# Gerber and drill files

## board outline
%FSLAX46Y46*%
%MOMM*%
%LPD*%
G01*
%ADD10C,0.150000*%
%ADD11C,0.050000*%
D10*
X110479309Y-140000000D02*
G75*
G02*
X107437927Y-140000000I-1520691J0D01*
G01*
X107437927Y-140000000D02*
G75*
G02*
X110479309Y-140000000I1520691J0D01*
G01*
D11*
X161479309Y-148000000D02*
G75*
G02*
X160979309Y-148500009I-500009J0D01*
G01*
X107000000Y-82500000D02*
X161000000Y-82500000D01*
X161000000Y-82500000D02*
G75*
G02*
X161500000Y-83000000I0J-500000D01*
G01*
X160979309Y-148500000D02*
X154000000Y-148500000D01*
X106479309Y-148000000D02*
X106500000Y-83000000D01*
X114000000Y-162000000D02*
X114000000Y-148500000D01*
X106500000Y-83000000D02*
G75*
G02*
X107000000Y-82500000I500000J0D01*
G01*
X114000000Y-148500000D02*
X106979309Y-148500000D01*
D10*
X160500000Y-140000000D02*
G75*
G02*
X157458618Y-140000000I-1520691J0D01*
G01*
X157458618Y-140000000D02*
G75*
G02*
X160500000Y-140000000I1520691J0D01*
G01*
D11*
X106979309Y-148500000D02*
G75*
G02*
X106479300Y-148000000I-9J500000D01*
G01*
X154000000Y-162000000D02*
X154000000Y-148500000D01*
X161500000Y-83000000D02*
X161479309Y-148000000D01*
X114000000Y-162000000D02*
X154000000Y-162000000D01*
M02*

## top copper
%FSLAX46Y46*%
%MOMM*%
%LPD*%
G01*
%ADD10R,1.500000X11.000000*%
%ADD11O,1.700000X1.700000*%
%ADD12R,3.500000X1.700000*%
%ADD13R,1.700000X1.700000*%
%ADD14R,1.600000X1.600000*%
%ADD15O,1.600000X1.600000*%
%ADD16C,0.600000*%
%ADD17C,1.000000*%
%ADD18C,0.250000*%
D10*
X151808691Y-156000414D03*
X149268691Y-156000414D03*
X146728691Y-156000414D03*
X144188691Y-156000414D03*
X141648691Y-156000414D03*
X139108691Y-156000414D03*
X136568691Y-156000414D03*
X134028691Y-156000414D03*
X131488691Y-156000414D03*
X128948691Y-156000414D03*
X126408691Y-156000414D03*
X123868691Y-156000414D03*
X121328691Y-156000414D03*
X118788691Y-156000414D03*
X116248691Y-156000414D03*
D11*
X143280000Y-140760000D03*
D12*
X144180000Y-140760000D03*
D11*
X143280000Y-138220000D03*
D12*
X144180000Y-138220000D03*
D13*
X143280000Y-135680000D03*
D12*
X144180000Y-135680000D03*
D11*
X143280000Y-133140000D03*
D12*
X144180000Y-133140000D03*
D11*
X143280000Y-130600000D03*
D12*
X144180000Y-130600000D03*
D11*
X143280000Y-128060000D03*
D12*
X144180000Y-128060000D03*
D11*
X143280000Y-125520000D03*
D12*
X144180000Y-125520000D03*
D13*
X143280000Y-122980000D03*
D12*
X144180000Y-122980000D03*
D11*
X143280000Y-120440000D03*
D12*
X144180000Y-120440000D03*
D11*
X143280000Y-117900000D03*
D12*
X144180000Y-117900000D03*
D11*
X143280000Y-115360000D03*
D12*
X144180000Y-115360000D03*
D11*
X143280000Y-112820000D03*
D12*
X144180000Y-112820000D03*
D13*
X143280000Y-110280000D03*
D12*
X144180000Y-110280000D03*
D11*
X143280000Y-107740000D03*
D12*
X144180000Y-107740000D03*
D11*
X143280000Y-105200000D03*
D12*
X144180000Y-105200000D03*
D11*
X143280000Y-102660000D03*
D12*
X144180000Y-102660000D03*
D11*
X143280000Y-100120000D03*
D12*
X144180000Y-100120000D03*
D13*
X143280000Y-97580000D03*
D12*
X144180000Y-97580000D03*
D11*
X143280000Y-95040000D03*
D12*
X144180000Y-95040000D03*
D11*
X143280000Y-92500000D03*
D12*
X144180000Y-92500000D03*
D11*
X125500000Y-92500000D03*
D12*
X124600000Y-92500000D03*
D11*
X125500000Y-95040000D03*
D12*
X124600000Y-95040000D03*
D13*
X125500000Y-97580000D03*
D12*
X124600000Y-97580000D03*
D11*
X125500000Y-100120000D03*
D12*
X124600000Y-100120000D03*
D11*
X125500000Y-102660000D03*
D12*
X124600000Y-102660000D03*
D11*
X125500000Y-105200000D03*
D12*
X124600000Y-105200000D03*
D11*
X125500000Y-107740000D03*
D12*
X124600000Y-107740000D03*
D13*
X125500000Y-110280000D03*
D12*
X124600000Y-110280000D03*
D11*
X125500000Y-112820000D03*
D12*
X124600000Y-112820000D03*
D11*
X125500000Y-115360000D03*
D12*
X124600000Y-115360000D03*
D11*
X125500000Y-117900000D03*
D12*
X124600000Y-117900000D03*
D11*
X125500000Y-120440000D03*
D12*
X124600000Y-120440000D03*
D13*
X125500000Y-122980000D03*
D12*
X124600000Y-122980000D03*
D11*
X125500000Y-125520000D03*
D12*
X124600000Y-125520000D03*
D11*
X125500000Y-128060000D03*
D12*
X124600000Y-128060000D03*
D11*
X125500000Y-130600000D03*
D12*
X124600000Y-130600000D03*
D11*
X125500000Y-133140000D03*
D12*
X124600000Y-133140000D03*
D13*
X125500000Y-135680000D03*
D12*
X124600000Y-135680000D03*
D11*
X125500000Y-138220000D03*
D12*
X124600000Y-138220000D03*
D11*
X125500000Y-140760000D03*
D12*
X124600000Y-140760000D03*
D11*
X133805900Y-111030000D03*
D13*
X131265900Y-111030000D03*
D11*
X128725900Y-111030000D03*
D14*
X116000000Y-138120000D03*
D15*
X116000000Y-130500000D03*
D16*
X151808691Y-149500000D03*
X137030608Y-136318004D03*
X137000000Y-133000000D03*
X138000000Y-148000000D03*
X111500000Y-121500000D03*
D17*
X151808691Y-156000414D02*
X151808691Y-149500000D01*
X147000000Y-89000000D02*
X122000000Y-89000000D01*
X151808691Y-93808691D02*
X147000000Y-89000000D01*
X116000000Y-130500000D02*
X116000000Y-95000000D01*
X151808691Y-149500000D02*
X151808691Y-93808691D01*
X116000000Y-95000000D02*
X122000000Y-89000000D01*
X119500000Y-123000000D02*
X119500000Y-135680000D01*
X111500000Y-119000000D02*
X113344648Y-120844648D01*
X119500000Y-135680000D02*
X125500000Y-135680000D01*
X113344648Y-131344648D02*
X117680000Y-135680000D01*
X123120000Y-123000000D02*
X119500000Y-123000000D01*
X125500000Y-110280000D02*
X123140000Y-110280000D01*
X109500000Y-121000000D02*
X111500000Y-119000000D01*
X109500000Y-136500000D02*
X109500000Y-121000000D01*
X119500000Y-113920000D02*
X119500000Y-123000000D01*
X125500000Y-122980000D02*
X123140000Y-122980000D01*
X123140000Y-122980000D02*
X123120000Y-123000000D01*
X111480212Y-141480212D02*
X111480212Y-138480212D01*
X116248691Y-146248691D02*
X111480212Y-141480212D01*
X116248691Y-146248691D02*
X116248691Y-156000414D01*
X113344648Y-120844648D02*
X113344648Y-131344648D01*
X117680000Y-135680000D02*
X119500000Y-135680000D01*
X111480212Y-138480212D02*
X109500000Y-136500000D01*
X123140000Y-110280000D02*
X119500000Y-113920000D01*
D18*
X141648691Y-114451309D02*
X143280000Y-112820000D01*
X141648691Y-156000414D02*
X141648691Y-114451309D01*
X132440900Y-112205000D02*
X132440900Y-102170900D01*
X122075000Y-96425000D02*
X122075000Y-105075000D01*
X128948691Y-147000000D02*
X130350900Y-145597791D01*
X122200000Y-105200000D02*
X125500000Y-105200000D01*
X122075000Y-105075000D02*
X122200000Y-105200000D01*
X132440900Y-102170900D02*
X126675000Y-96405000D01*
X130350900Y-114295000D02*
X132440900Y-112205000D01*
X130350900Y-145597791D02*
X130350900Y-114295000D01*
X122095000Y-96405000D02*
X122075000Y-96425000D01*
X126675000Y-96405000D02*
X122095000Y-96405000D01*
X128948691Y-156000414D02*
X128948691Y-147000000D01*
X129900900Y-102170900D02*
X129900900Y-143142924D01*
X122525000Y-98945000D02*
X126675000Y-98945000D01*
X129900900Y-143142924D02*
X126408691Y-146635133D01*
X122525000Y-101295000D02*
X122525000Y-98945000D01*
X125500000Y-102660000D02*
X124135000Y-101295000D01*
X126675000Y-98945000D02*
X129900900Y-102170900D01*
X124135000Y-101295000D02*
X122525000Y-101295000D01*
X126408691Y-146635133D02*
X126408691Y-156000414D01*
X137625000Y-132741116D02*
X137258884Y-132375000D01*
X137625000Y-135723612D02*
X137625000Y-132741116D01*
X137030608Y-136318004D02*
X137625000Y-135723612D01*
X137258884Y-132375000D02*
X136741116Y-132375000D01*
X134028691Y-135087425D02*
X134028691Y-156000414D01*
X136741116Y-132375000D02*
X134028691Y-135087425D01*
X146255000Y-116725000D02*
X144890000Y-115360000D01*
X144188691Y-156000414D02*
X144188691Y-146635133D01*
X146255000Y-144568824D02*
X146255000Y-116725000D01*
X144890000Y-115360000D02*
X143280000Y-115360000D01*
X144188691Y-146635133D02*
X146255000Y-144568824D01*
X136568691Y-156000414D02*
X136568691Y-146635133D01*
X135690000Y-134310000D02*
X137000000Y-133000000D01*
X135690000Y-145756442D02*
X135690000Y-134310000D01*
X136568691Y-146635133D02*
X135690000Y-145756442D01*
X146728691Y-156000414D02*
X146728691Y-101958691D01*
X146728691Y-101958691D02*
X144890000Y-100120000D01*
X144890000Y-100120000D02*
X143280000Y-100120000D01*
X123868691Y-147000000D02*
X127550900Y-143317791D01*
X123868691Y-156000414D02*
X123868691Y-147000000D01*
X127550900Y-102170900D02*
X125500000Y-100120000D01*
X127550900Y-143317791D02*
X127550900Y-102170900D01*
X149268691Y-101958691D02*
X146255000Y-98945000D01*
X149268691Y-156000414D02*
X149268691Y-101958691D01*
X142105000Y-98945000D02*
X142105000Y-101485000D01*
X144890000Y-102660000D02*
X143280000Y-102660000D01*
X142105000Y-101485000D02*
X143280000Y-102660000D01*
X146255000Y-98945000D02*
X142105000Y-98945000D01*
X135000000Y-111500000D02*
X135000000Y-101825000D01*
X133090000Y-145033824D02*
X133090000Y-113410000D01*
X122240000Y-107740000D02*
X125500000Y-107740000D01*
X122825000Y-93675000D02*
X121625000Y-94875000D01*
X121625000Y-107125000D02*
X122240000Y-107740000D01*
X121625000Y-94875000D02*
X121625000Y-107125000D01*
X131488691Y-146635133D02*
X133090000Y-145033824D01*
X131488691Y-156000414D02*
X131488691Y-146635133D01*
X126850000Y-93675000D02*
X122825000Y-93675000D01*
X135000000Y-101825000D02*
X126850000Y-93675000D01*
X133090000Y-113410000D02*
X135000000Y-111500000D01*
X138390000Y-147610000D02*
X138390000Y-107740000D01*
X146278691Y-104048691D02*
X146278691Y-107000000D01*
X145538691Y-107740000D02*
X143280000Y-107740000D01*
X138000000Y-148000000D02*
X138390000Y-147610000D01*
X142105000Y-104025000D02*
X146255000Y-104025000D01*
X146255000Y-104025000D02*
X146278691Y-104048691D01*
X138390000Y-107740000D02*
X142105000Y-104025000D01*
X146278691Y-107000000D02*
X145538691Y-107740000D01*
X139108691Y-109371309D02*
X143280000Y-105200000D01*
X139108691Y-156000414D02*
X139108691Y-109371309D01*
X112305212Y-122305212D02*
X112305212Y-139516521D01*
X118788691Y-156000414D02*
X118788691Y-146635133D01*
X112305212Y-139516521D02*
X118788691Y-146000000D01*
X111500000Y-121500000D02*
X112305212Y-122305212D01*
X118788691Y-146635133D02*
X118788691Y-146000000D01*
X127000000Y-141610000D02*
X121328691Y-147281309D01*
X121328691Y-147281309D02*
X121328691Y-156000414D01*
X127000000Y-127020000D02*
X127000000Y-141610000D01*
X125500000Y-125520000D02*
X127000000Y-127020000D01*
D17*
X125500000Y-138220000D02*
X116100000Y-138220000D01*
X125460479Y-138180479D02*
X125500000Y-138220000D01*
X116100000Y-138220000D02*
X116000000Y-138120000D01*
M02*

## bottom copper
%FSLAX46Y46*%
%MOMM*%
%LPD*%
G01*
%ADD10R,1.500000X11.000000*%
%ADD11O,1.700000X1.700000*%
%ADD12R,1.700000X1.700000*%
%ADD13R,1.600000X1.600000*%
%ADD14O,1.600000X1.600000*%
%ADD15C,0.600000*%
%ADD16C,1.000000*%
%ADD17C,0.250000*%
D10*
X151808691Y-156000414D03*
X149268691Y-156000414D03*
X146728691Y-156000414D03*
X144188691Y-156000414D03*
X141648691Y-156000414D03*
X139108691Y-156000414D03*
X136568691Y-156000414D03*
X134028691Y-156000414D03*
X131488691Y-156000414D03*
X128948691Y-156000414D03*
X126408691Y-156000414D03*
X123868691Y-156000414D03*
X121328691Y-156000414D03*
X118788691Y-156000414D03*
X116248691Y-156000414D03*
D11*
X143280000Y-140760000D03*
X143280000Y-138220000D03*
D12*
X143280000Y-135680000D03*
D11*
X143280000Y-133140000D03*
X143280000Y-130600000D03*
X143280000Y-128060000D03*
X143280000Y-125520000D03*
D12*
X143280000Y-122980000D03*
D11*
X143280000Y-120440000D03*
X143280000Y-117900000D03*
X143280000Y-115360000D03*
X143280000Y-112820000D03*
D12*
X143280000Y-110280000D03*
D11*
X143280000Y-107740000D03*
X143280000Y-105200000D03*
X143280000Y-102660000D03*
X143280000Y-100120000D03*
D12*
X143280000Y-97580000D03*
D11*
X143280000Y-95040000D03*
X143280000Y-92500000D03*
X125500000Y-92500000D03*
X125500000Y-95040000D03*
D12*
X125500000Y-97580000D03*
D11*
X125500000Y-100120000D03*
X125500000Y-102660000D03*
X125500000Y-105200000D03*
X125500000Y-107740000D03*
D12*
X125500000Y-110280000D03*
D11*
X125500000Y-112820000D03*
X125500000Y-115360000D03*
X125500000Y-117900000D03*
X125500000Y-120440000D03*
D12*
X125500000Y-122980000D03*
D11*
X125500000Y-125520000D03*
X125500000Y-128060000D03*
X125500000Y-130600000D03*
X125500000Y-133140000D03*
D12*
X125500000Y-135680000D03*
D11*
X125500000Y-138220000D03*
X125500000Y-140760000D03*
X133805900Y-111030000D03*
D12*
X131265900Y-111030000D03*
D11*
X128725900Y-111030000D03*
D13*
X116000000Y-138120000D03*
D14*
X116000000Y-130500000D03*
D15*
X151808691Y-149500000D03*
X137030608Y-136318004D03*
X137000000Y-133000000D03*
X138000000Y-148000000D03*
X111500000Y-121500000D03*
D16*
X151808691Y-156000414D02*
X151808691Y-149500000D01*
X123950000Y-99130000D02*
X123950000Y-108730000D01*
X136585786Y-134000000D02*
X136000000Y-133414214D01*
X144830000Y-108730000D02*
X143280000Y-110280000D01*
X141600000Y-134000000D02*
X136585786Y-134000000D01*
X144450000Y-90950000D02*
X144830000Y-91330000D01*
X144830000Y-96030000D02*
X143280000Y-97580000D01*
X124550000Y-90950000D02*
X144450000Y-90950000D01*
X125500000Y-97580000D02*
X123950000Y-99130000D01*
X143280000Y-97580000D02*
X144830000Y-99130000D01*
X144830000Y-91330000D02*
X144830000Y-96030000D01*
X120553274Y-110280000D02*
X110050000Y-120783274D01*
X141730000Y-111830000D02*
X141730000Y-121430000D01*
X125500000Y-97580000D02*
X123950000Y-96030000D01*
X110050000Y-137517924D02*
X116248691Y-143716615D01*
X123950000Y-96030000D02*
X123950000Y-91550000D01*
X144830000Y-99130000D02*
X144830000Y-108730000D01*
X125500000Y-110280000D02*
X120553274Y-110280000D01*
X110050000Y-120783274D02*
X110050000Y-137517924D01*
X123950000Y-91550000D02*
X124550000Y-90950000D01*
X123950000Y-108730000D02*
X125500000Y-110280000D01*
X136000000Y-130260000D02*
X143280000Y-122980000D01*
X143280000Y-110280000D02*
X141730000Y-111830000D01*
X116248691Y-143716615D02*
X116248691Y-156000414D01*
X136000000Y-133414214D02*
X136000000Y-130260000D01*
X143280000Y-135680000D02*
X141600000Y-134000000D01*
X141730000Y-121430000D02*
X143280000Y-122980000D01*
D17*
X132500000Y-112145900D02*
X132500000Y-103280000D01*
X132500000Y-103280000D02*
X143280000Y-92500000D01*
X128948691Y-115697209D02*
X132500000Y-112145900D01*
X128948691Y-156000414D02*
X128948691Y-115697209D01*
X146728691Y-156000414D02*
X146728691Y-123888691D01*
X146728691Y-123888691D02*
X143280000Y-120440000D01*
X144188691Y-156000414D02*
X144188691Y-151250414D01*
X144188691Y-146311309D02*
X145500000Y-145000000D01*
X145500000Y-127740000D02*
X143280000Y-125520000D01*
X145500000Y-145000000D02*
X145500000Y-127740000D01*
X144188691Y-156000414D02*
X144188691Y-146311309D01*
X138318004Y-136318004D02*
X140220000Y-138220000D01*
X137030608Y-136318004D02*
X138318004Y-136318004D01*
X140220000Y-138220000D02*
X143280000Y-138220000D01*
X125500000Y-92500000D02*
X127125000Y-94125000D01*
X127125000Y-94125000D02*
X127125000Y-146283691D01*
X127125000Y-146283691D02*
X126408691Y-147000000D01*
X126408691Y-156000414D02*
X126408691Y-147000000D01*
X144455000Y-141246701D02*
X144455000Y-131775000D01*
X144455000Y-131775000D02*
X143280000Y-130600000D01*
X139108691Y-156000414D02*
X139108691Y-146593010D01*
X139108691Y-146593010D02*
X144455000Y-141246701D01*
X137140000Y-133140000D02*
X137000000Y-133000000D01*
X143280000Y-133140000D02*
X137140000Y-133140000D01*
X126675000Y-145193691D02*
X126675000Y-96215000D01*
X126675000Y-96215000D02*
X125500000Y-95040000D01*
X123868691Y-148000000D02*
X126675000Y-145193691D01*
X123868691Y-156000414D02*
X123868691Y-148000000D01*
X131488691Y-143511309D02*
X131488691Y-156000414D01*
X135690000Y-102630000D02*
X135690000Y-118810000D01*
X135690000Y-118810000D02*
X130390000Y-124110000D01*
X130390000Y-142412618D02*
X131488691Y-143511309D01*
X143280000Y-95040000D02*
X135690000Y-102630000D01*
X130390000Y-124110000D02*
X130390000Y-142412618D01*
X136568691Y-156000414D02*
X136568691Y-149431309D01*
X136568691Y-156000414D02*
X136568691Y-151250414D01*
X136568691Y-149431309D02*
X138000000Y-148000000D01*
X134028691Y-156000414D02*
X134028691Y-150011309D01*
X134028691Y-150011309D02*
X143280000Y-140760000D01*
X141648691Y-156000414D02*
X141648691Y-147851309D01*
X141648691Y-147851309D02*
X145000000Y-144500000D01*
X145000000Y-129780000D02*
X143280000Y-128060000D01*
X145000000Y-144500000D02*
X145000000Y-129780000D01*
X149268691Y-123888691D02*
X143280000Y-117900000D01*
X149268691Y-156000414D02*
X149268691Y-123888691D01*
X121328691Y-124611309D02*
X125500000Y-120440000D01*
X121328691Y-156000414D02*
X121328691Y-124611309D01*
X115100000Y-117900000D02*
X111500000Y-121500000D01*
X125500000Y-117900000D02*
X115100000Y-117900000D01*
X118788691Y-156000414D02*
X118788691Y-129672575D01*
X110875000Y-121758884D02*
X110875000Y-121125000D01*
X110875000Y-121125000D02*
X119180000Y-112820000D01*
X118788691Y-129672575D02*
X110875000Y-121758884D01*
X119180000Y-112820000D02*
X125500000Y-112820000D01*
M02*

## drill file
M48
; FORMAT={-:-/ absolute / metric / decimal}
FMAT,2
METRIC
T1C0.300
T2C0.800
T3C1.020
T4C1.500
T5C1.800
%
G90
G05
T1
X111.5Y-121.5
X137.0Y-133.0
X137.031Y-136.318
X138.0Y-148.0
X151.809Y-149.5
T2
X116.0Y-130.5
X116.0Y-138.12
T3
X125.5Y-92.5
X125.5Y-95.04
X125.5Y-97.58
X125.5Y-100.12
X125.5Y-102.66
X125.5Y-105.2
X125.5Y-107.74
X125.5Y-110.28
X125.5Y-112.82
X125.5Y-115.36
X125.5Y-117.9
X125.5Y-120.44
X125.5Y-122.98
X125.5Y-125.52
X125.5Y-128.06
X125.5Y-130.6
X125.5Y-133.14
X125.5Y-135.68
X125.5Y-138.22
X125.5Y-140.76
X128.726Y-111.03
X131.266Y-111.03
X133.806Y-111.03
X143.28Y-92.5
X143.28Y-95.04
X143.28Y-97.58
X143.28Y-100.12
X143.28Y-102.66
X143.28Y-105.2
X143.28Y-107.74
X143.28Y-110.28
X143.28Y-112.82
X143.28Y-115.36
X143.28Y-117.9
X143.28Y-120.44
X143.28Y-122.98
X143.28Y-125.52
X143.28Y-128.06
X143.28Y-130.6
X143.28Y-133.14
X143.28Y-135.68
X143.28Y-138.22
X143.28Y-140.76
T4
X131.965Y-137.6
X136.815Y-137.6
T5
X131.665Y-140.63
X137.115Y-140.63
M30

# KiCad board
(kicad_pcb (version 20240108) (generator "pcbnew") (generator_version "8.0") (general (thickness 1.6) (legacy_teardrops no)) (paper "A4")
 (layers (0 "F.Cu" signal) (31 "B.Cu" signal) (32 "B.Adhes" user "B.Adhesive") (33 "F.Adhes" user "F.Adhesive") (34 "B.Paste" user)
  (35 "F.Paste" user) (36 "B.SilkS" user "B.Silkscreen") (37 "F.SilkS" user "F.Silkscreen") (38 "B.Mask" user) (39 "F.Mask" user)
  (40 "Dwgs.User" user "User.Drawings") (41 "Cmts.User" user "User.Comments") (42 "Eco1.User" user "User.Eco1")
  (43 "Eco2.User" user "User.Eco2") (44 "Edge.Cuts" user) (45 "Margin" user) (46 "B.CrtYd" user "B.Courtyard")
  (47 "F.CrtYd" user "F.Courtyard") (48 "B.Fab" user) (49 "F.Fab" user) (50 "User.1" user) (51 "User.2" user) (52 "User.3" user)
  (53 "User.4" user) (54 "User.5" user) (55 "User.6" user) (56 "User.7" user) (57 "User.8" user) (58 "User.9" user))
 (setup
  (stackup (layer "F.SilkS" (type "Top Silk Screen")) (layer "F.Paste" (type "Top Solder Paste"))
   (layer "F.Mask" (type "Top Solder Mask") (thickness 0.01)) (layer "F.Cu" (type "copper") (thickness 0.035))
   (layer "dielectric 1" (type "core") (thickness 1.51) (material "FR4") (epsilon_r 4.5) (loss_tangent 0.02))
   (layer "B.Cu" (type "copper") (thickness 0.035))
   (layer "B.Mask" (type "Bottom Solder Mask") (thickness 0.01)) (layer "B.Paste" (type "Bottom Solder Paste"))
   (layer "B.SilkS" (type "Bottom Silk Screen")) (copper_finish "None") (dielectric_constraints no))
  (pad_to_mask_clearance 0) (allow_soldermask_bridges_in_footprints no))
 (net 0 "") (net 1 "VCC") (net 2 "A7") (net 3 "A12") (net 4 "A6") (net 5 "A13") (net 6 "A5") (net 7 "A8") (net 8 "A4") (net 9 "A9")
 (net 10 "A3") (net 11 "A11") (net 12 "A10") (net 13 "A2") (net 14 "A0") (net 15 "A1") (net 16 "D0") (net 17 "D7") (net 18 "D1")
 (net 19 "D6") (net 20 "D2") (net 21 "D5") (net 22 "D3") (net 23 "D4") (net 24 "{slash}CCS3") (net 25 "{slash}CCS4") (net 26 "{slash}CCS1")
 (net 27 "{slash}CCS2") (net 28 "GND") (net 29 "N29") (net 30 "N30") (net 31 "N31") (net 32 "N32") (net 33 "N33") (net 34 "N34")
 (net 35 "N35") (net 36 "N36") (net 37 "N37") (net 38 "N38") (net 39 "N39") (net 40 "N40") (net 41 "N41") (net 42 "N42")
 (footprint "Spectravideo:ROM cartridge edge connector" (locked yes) (layer "F.Cu") (at 134.028691 156.127414)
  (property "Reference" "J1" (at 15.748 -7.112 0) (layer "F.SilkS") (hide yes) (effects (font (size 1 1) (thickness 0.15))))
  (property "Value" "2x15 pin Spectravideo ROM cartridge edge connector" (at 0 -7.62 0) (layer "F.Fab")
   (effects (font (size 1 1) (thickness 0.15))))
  (pad "1" connect rect (at 17.78 -0.127) (size 1.5 11) (layers "B.Cu" "B.Mask") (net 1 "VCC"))
  (pad "2" connect rect (at 17.78 -0.127) (size 1.5 11) (layers "F.Cu" "F.Mask") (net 1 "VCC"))
  (pad "3" connect rect (at 15.24 -0.127) (size 1.5 11) (layers "B.Cu" "B.Mask") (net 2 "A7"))
  (pad "4" connect rect (at 15.24 -0.127) (size 1.5 11) (layers "F.Cu" "F.Mask") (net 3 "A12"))
  (pad "5" connect rect (at 12.7 -0.127) (size 1.5 11) (layers "B.Cu" "B.Mask") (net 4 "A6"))
  (pad "6" connect rect (at 12.7 -0.127) (size 1.5 11) (layers "F.Cu" "F.Mask") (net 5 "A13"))
  (pad "7" connect rect (at 10.16 -0.127) (size 1.5 11) (layers "B.Cu" "B.Mask") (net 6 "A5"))
  (pad "8" connect rect (at 10.16 -0.127) (size 1.5 11) (layers "F.Cu" "F.Mask") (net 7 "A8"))
  (pad "9" connect rect (at 7.62 -0.127) (size 1.5 11) (layers "B.Cu" "B.Mask") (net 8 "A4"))
  (pad "10" connect rect (at 7.62 -0.127) (size 1.5 11) (layers "F.Cu" "F.Mask") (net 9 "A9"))
  (pad "11" connect rect (at 5.08 -0.127) (size 1.5 11) (layers "B.Cu" "B.Mask") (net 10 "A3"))
  (pad "12" connect rect (at 5.08 -0.127) (size 1.5 11) (layers "F.Cu" "F.Mask") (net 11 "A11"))
  (pad "13" connect rect (at 2.54 -0.127) (size 1.5 11) (layers "B.Cu" "B.Mask") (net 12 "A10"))
  (pad "14" connect rect (at 2.54 -0.127) (size 1.5 11) (layers "F.Cu" "F.Mask") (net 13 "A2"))
  (pad "15" connect rect (at 0 -0.127) (size 1.5 11) (layers "B.Cu" "B.Mask") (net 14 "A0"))
  (pad "16" connect rect (at 0 -0.127) (size 1.5 11) (layers "F.Cu" "F.Mask") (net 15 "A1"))
  (pad "17" connect rect (at -2.54 -0.127) (size 1.5 11) (layers "B.Cu" "B.Mask") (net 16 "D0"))
  (pad "18" connect rect (at -2.54 -0.127) (size 1.5 11) (layers "F.Cu" "F.Mask") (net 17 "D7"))
  (pad "19" connect rect (at -5.08 -0.127) (size 1.5 11) (layers "B.Cu" "B.Mask") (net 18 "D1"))
  (pad "20" connect rect (at -5.08 -0.127) (size 1.5 11) (layers "F.Cu" "F.Mask") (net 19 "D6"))
  (pad "21" connect rect (at -7.62 -0.127) (size 1.5 11) (layers "B.Cu" "B.Mask") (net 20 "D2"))
  (pad "22" connect rect (at -7.62 -0.127) (size 1.5 11) (layers "F.Cu" "F.Mask") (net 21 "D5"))
  (pad "23" connect rect (at -10.16 -0.127) (size 1.5 11) (layers "B.Cu" "B.Mask") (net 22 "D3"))
  (pad "24" connect rect (at -10.16 -0.127) (size 1.5 11) (layers "F.Cu" "F.Mask") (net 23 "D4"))
  (pad "25" connect rect (at -12.7 -0.127) (size 1.5 11) (layers "B.Cu" "B.Mask") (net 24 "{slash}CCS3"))
  (pad "26" connect rect (at -12.7 -0.127) (size 1.5 11) (layers "F.Cu" "F.Mask") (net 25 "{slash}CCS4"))
  (pad "27" connect rect (at -15.24 -0.127) (size 1.5 11) (layers "B.Cu" "B.Mask") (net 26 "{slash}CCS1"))
  (pad "28" connect rect (at -15.24 -0.127) (size 1.5 11) (layers "F.Cu" "F.Mask") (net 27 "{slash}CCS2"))
  (pad "29" connect rect (at -17.78 -0.127) (size 1.5 11) (layers "B.Cu" "B.Mask") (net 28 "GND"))
  (pad "30" connect rect (at -17.78 -0.127) (size 1.5 11) (layers "F.Cu" "F.Mask") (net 28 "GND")))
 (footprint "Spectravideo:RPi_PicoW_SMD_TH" (layer "F.Cu") (at 134.39 116.63 180)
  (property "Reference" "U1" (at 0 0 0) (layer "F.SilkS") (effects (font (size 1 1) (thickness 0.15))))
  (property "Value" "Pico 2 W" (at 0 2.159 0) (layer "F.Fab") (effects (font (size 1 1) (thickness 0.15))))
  (pad "" np_thru_hole oval (at -2.725 -24 180) (size 1.8 1.8) (drill 1.8) (layers "*.Cu" "*.Mask"))
  (pad "" np_thru_hole oval (at -2.425 -20.97 180) (size 1.5 1.5) (drill 1.5) (layers "*.Cu" "*.Mask"))
  (pad "" np_thru_hole oval (at 2.425 -20.97 180) (size 1.5 1.5) (drill 1.5) (layers "*.Cu" "*.Mask"))
  (pad "" np_thru_hole oval (at 2.725 -24 180) (size 1.8 1.8) (drill 1.8) (layers "*.Cu" "*.Mask"))
  (pad "1" thru_hole oval (at -8.89 -24.13 180) (size 1.7 1.7) (drill 1.02) (layers "*.Cu" "*.Mask") (remove_unused_layers no) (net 14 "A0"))
  (pad "1" smd rect (at -8.89 -24.13 180) (size 3.5 1.7) (drill (offset -0.9 0)) (layers "F.Cu" "F.Mask") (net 14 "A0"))
  (pad "2" thru_hole oval (at -8.89 -21.59 180) (size 1.7 1.7) (drill 1.02) (layers "*.Cu" "*.Mask") (remove_unused_layers no) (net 15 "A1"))
  (pad "2" smd rect (at -8.89 -21.59 180) (size 3.5 1.7) (drill (offset -0.9 0)) (layers "F.Cu" "F.Mask") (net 15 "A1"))
  (pad "3" thru_hole rect (at -8.89 -19.05 180) (size 1.7 1.7) (drill 1.02) (layers "*.Cu" "*.Mask") (remove_unused_layers no)
   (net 28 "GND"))
  (pad "3" smd rect (at -8.89 -19.05 180) (size 3.5 1.7) (drill (offset -0.9 0)) (layers "F.Cu" "F.Mask") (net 28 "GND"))
  (pad "4" thru_hole oval (at -8.89 -16.51 180) (size 1.7 1.7) (drill 1.02) (layers "*.Cu" "*.Mask") (remove_unused_layers no) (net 13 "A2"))
  (pad "4" smd rect (at -8.89 -16.51 180) (size 3.5 1.7) (drill (offset -0.9 0)) (layers "F.Cu" "F.Mask") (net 13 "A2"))
  (pad "5" thru_hole oval (at -8.89 -13.97 180) (size 1.7 1.7) (drill 1.02) (layers "*.Cu" "*.Mask") (remove_unused_layers no) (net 10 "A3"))
  (pad "5" smd rect (at -8.89 -13.97 180) (size 3.5 1.7) (drill (offset -0.9 0)) (layers "F.Cu" "F.Mask") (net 10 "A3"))
  (pad "6" thru_hole oval (at -8.89 -11.43 180) (size 1.7 1.7) (drill 1.02) (layers "*.Cu" "*.Mask") (remove_unused_layers no) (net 8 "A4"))
  (pad "6" smd rect (at -8.89 -11.43 180) (size 3.5 1.7) (drill (offset -0.9 0)) (layers "F.Cu" "F.Mask") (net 8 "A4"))
  (pad "7" thru_hole oval (at -8.89 -8.89 180) (size 1.7 1.7) (drill 1.02) (layers "*.Cu" "*.Mask") (remove_unused_layers no) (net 6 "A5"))
  (pad "7" smd rect (at -8.89 -8.89 180) (size 3.5 1.7) (drill (offset -0.9 0)) (layers "F.Cu" "F.Mask") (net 6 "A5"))
  (pad "8" thru_hole rect (at -8.89 -6.35 180) (size 1.7 1.7) (drill 1.02) (layers "*.Cu" "*.Mask") (remove_unused_layers no) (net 28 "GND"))
  (pad "8" smd rect (at -8.89 -6.35 180) (size 3.5 1.7) (drill (offset -0.9 0)) (layers "F.Cu" "F.Mask") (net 28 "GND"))
  (pad "9" thru_hole oval (at -8.89 -3.81 180) (size 1.7 1.7) (drill 1.02) (layers "*.Cu" "*.Mask") (remove_unused_layers no) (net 4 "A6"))
  (pad "9" smd rect (at -8.89 -3.81 180) (size 3.5 1.7) (drill (offset -0.9 0)) (layers "F.Cu" "F.Mask") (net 4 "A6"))
  (pad "10" thru_hole oval (at -8.89 -1.27 180) (size 1.7 1.7) (drill 1.02) (layers "*.Cu" "*.Mask") (remove_unused_layers no) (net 2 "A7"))
  (pad "10" smd rect (at -8.89 -1.27 180) (size 3.5 1.7) (drill (offset -0.9 0)) (layers "F.Cu" "F.Mask") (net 2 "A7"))
  (pad "11" thru_hole oval (at -8.89 1.27 180) (size 1.7 1.7) (drill 1.02) (layers "*.Cu" "*.Mask") (remove_unused_layers no) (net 7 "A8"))
  (pad "11" smd rect (at -8.89 1.27 180) (size 3.5 1.7) (drill (offset -0.9 0)) (layers "F.Cu" "F.Mask") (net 7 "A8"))
  (pad "12" thru_hole oval (at -8.89 3.81 180) (size 1.7 1.7) (drill 1.02) (layers "*.Cu" "*.Mask") (remove_unused_layers no) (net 9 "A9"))
  (pad "12" smd rect (at -8.89 3.81 180) (size 3.5 1.7) (drill (offset -0.9 0)) (layers "F.Cu" "F.Mask") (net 9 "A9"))
  (pad "13" thru_hole rect (at -8.89 6.35 180) (size 1.7 1.7) (drill 1.02) (layers "*.Cu" "*.Mask") (remove_unused_layers no) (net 28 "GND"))
  (pad "13" smd rect (at -8.89 6.35 180) (size 3.5 1.7) (drill (offset -0.9 0)) (layers "F.Cu" "F.Mask") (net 28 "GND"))
  (pad "14" thru_hole oval (at -8.89 8.89 180) (size 1.7 1.7) (drill 1.02) (layers "*.Cu" "*.Mask") (remove_unused_layers no) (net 12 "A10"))
  (pad "14" smd rect (at -8.89 8.89 180) (size 3.5 1.7) (drill (offset -0.9 0)) (layers "F.Cu" "F.Mask") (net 12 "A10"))
  (pad "15" thru_hole oval (at -8.89 11.43 180) (size 1.7 1.7) (drill 1.02) (layers "*.Cu" "*.Mask") (remove_unused_layers no)
   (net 11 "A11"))
  (pad "15" smd rect (at -8.89 11.43 180) (size 3.5 1.7) (drill (offset -0.9 0)) (layers "F.Cu" "F.Mask") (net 11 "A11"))
  (pad "16" thru_hole oval (at -8.89 13.97 180) (size 1.7 1.7) (drill 1.02) (layers "*.Cu" "*.Mask") (remove_unused_layers no) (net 3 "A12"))
  (pad "16" smd rect (at -8.89 13.97 180) (size 3.5 1.7) (drill (offset -0.9 0)) (layers "F.Cu" "F.Mask") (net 3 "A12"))
  (pad "17" thru_hole oval (at -8.89 16.51 180) (size 1.7 1.7) (drill 1.02) (layers "*.Cu" "*.Mask") (remove_unused_layers no) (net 5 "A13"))
  (pad "17" smd rect (at -8.89 16.51 180) (size 3.5 1.7) (drill (offset -0.9 0)) (layers "F.Cu" "F.Mask") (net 5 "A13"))
  (pad "18" thru_hole rect (at -8.89 19.05 180) (size 1.7 1.7) (drill 1.02) (layers "*.Cu" "*.Mask") (remove_unused_layers no)
   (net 28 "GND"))
  (pad "18" smd rect (at -8.89 19.05 180) (size 3.5 1.7) (drill (offset -0.9 0)) (layers "F.Cu" "F.Mask") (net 28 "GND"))
  (pad "19" thru_hole oval (at -8.89 21.59 180) (size 1.7 1.7) (drill 1.02) (layers "*.Cu" "*.Mask") (remove_unused_layers no) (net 16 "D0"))
  (pad "19" smd rect (at -8.89 21.59 180) (size 3.5 1.7) (drill (offset -0.9 0)) (layers "F.Cu" "F.Mask") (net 16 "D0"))
  (pad "20" thru_hole oval (at -8.89 24.13 180) (size 1.7 1.7) (drill 1.02) (layers "*.Cu" "*.Mask") (remove_unused_layers no) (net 18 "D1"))
  (pad "20" smd rect (at -8.89 24.13 180) (size 3.5 1.7) (drill (offset -0.9 0)) (layers "F.Cu" "F.Mask") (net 18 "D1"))
  (pad "21" thru_hole oval (at 8.89 24.13 180) (size 1.7 1.7) (drill 1.02) (layers "*.Cu" "*.Mask") (remove_unused_layers no) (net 20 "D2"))
  (pad "21" smd rect (at 8.89 24.13 180) (size 3.5 1.7) (drill (offset 0.9 0)) (layers "F.Cu" "F.Mask") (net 20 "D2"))
  (pad "22" thru_hole oval (at 8.89 21.59 180) (size 1.7 1.7) (drill 1.02) (layers "*.Cu" "*.Mask") (remove_unused_layers no) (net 22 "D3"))
  (pad "22" smd rect (at 8.89 21.59 180) (size 3.5 1.7) (drill (offset 0.9 0)) (layers "F.Cu" "F.Mask") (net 22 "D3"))
  (pad "23" thru_hole rect (at 8.89 19.05 180) (size 1.7 1.7) (drill 1.02) (layers "*.Cu" "*.Mask") (remove_unused_layers no) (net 28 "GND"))
  (pad "23" smd rect (at 8.89 19.05 180) (size 3.5 1.7) (drill (offset 0.9 0)) (layers "F.Cu" "F.Mask") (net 28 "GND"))
  (pad "24" thru_hole oval (at 8.89 16.51 180) (size 1.7 1.7) (drill 1.02) (layers "*.Cu" "*.Mask") (remove_unused_layers no) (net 23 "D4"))
  (pad "24" smd rect (at 8.89 16.51 180) (size 3.5 1.7) (drill (offset 0.9 0)) (layers "F.Cu" "F.Mask") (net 23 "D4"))
  (pad "25" thru_hole oval (at 8.89 13.97 180) (size 1.7 1.7) (drill 1.02) (layers "*.Cu" "*.Mask") (remove_unused_layers no) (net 21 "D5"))
  (pad "25" smd rect (at 8.89 13.97 180) (size 3.5 1.7) (drill (offset 0.9 0)) (layers "F.Cu" "F.Mask") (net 21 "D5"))
  (pad "26" thru_hole oval (at 8.89 11.43 180) (size 1.7 1.7) (drill 1.02) (layers "*.Cu" "*.Mask") (remove_unused_layers no) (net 19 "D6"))
  (pad "26" smd rect (at 8.89 11.43 180) (size 3.5 1.7) (drill (offset 0.9 0)) (layers "F.Cu" "F.Mask") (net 19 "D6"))
  (pad "27" thru_hole oval (at 8.89 8.89 180) (size 1.7 1.7) (drill 1.02) (layers "*.Cu" "*.Mask") (remove_unused_layers no) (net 17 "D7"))
  (pad "27" smd rect (at 8.89 8.89 180) (size 3.5 1.7) (drill (offset 0.9 0)) (layers "F.Cu" "F.Mask") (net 17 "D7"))
  (pad "28" thru_hole rect (at 8.89 6.35 180) (size 1.7 1.7) (drill 1.02) (layers "*.Cu" "*.Mask") (remove_unused_layers no) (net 28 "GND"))
  (pad "28" smd rect (at 8.89 6.35 180) (size 3.5 1.7) (drill (offset 0.9 0)) (layers "F.Cu" "F.Mask") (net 28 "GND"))
  (pad "29" thru_hole oval (at 8.89 3.81 180) (size 1.7 1.7) (drill 1.02) (layers "*.Cu" "*.Mask") (remove_unused_layers no)
   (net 26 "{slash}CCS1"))
  (pad "29" smd rect (at 8.89 3.81 180) (size 3.5 1.7) (drill (offset 0.9 0)) (layers "F.Cu" "F.Mask") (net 26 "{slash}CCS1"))
  (pad "30" thru_hole oval (at 8.89 1.27 180) (size 1.7 1.7) (drill 1.02) (layers "*.Cu" "*.Mask") (remove_unused_layers no) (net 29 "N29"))
  (pad "30" smd rect (at 8.89 1.27 180) (size 3.5 1.7) (drill (offset 0.9 0)) (layers "F.Cu" "F.Mask") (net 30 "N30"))
  (pad "31" thru_hole oval (at 8.89 -1.27 180) (size 1.7 1.7) (drill 1.02) (layers "*.Cu" "*.Mask") (remove_unused_layers no)
   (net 27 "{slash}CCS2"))
  (pad "31" smd rect (at 8.89 -1.27 180) (size 3.5 1.7) (drill (offset 0.9 0)) (layers "F.Cu" "F.Mask") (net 27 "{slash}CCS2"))
  (pad "32" thru_hole oval (at 8.89 -3.81 180) (size 1.7 1.7) (drill 1.02) (layers "*.Cu" "*.Mask") (remove_unused_layers no)
   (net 24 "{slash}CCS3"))
  (pad "32" smd rect (at 8.89 -3.81 180) (size 3.5 1.7) (drill (offset 0.9 0)) (layers "F.Cu" "F.Mask") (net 24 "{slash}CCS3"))
  (pad "33" thru_hole rect (at 8.89 -6.35 180) (size 1.7 1.7) (drill 1.02) (layers "*.Cu" "*.Mask") (remove_unused_layers no) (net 28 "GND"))
  (pad "33" smd rect (at 8.89 -6.35 180) (size 3.5 1.7) (drill (offset 0.9 0)) (layers "F.Cu" "F.Mask") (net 28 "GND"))
  (pad "34" thru_hole oval (at 8.89 -8.89 180) (size 1.7 1.7) (drill 1.02) (layers "*.Cu" "*.Mask") (remove_unused_layers no)
   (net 25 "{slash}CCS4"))
  (pad "34" smd rect (at 8.89 -8.89 180) (size 3.5 1.7) (drill (offset 0.9 0)) (layers "F.Cu" "F.Mask") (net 25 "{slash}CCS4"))
  (pad "35" thru_hole oval (at 8.89 -11.43 180) (size 1.7 1.7) (drill 1.02) (layers "*.Cu" "*.Mask") (remove_unused_layers no)
   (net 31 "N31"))
  (pad "35" smd rect (at 8.89 -11.43 180) (size 3.5 1.7) (drill (offset 0.9 0)) (layers "F.Cu" "F.Mask") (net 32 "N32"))
  (pad "36" thru_hole oval (at 8.89 -13.97 180) (size 1.7 1.7) (drill 1.02) (layers "*.Cu" "*.Mask") (remove_unused_layers no)
   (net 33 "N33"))
  (pad "36" smd rect (at 8.89 -13.97 180) (size 3.5 1.7) (drill (offset 0.9 0)) (layers "F.Cu" "F.Mask") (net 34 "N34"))
  (pad "37" thru_hole oval (at 8.89 -16.51 180) (size 1.7 1.7) (drill 1.02) (layers "*.Cu" "*.Mask") (remove_unused_layers no)
   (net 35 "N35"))
  (pad "37" smd rect (at 8.89 -16.51 180) (size 3.5 1.7) (drill (offset 0.9 0)) (layers "F.Cu" "F.Mask") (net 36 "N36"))
  (pad "38" thru_hole rect (at 8.89 -19.05 180) (size 1.7 1.7) (drill 1.02) (layers "*.Cu" "*.Mask") (remove_unused_layers no)
   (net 28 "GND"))
  (pad "38" smd rect (at 8.89 -19.05 180) (size 3.5 1.7) (drill (offset 0.9 0)) (layers "F.Cu" "F.Mask") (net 28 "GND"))
  (pad "39" thru_hole oval (at 8.89 -21.59 180) (size 1.7 1.7) (drill 1.02) (layers "*.Cu" "*.Mask") (remove_unused_layers no)
   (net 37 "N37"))
  (pad "39" smd rect (at 8.89 -21.59 180) (size 3.5 1.7) (drill (offset 0.9 0)) (layers "F.Cu" "F.Mask") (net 37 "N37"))
  (pad "40" thru_hole oval (at 8.89 -24.13 180) (size 1.7 1.7) (drill 1.02) (layers "*.Cu" "*.Mask") (remove_unused_layers no)
   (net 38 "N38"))
  (pad "40" smd rect (at 8.89 -24.13 180) (size 3.5 1.7) (drill (offset 0.9 0)) (layers "F.Cu" "F.Mask") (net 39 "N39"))
  (pad "41" thru_hole oval (at 0.5841 5.6 180) (size 1.7 1.7) (drill 1.02) (layers "*.Cu" "*.Mask") (remove_unused_layers no) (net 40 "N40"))
  (pad "42" thru_hole rect (at 3.1241 5.6 180) (size 1.7 1.7) (drill 1.02) (layers "*.Cu" "*.Mask") (remove_unused_layers no) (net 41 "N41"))
  (pad "43" thru_hole oval (at 5.6641 5.6 180) (size 1.7 1.7) (drill 1.02) (layers "*.Cu" "*.Mask") (remove_unused_layers no) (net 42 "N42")))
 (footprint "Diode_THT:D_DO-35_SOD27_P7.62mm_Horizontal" (layer "F.Cu") (at 116 138.12 90)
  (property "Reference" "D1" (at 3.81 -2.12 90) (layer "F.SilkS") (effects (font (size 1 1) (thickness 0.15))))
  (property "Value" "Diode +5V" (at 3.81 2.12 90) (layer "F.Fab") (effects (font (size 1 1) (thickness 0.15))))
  (pad "1" thru_hole rect (at 0 0 90) (size 1.6 1.6) (drill 0.8) (layers "*.Cu" "*.Mask") (remove_unused_layers no) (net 37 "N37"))
  (pad "2" thru_hole oval (at 7.62 0 90) (size 1.6 1.6) (drill 0.8) (layers "*.Cu" "*.Mask") (remove_unused_layers no) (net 1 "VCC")))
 (gr_circle (center 108.958618 140) (end 110.479309 140) (stroke (width 0.15) (type solid)) (fill none) (layer "Edge.Cuts"))
 (gr_arc (start 161.479309 148) (mid 161.332862 148.353553) (end 160.979309 148.5) (stroke (width 0.05) (type solid)) (layer "Edge.Cuts"))
 (gr_line (start 107 82.5) (end 161 82.5) (stroke (width 0.05) (type solid)) (layer "Edge.Cuts"))
 (gr_arc (start 161 82.5) (mid 161.353548 82.64645) (end 161.5 83) (stroke (width 0.05) (type solid)) (layer "Edge.Cuts"))
 (gr_line (start 160.979309 148.5) (end 154 148.5) (stroke (width 0.05) (type solid)) (layer "Edge.Cuts"))
 (gr_line (start 106.479309 148) (end 106.5 83) (stroke (width 0.05) (type solid)) (layer "Edge.Cuts"))
 (gr_line (start 114 162) (end 114 148.5) (stroke (width 0.05) (type solid)) (layer "Edge.Cuts"))
 (gr_arc (start 106.5 83) (mid 106.646447 82.64645) (end 107 82.5) (stroke (width 0.05) (type solid)) (layer "Edge.Cuts"))
 (gr_line (start 114 148.5) (end 106.979309 148.5) (stroke (width 0.05) (type solid)) (layer "Edge.Cuts"))
 (gr_circle (center 158.979309 140) (end 160.5 140) (stroke (width 0.15) (type solid)) (fill none) (layer "Edge.Cuts"))
 (gr_arc (start 106.979309 148.5) (mid 106.625756 148.353553) (end 106.479309 148) (stroke (width 0.05) (type solid)) (layer "Edge.Cuts"))
 (gr_line (start 154 162) (end 154 148.5) (stroke (width 0.05) (type solid)) (layer "Edge.Cuts"))
 (gr_line (start 161.5 83) (end 161.479309 148) (stroke (width 0.05) (type solid)) (layer "Edge.Cuts"))
 (gr_line (start 114 162) (end 154 162) (stroke (width 0.05) (type solid)) (layer "Edge.Cuts"))
 (segment (start 151.808691 156.000414) (end 151.808691 149.5) (width 1) (layer "F.Cu") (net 1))
 (segment (start 147 89) (end 122 89) (width 1) (layer "F.Cu") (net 1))
 (segment (start 151.808691 93.808691) (end 147 89) (width 1) (layer "F.Cu") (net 1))
 (segment (start 116 130.5) (end 116 95) (width 1) (layer "F.Cu") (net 1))
 (segment (start 151.808691 149.5) (end 151.808691 93.808691) (width 1) (layer "F.Cu") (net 1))
 (segment (start 116 95) (end 122 89) (width 1) (layer "F.Cu") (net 1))
 (via (at 151.808691 149.5) (size 0.6) (drill 0.3) (layers "F.Cu" "B.Cu") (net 1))
 (segment (start 151.808691 156.000414) (end 151.808691 149.5) (width 1) (layer "B.Cu") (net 1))
 (segment (start 119.5 123) (end 119.5 135.68) (width 1) (layer "F.Cu") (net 28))
 (segment (start 111.5 119) (end 113.344648 120.844648) (width 1) (layer "F.Cu") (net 28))
 (segment (start 119.5 135.68) (end 125.5 135.68) (width 1) (layer "F.Cu") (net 28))
 (segment (start 113.344648 131.344648) (end 117.68 135.68) (width 1) (layer "F.Cu") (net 28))
 (segment (start 123.12 123) (end 119.5 123) (width 1) (layer "F.Cu") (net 28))
 (segment (start 125.5 110.28) (end 123.14 110.28) (width 1) (layer "F.Cu") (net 28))
 (segment (start 109.5 121) (end 111.5 119) (width 1) (layer "F.Cu") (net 28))
 (segment (start 109.5 136.5) (end 109.5 121) (width 1) (layer "F.Cu") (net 28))
 (segment (start 119.5 113.92) (end 119.5 123) (width 1) (layer "F.Cu") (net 28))
 (segment (start 125.5 122.98) (end 123.14 122.98) (width 1) (layer "F.Cu") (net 28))
 (segment (start 123.14 122.98) (end 123.12 123) (width 1) (layer "F.Cu") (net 28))
 (segment (start 111.480212 141.480212) (end 111.480212 138.480212) (width 1) (layer "F.Cu") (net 28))
 (segment (start 116.248691 146.248691) (end 111.480212 141.480212) (width 1) (layer "F.Cu") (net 28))
 (segment (start 116.248691 146.248691) (end 116.248691 156.000414) (width 1) (layer "F.Cu") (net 28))
 (segment (start 113.344648 120.844648) (end 113.344648 131.344648) (width 1) (layer "F.Cu") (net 28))
 (segment (start 117.68 135.68) (end 119.5 135.68) (width 1) (layer "F.Cu") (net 28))
 (segment (start 111.480212 138.480212) (end 109.5 136.5) (width 1) (layer "F.Cu") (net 28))
 (segment (start 123.14 110.28) (end 119.5 113.92) (width 1) (layer "F.Cu") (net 28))
 (segment (start 123.95 99.13) (end 123.95 108.73) (width 1) (layer "B.Cu") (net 28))
 (segment (start 136.585786 134) (end 136 133.414214) (width 1) (layer "B.Cu") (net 28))
 (segment (start 144.83 108.73) (end 143.28 110.28) (width 1) (layer "B.Cu") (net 28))
 (segment (start 141.6 134) (end 136.585786 134) (width 1) (layer "B.Cu") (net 28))
 (segment (start 144.45 90.95) (end 144.83 91.33) (width 1) (layer "B.Cu") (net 28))
 (segment (start 144.83 96.03) (end 143.28 97.58) (width 1) (layer "B.Cu") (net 28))
 (segment (start 124.55 90.95) (end 144.45 90.95) (width 1) (layer "B.Cu") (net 28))
 (segment (start 125.5 97.58) (end 123.95 99.13) (width 1) (layer "B.Cu") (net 28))
 (segment (start 143.28 97.58) (end 144.83 99.13) (width 1) (layer "B.Cu") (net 28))
 (segment (start 144.83 91.33) (end 144.83 96.03) (width 1) (layer "B.Cu") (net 28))
 (segment (start 120.553274 110.28) (end 110.05 120.783274) (width 1) (layer "B.Cu") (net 28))
 (segment (start 141.73 111.83) (end 141.73 121.43) (width 1) (layer "B.Cu") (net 28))
 (segment (start 125.5 97.58) (end 123.95 96.03) (width 1) (layer "B.Cu") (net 28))
 (segment (start 110.05 137.517924) (end 116.248691 143.716615) (width 1) (layer "B.Cu") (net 28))
 (segment (start 123.95 96.03) (end 123.95 91.55) (width 1) (layer "B.Cu") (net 28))
 (segment (start 144.83 99.13) (end 144.83 108.73) (width 1) (layer "B.Cu") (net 28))
 (segment (start 125.5 110.28) (end 120.553274 110.28) (width 1) (layer "B.Cu") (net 28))
 (segment (start 110.05 120.783274) (end 110.05 137.517924) (width 1) (layer "B.Cu") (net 28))
 (segment (start 123.95 91.55) (end 124.55 90.95) (width 1) (layer "B.Cu") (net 28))
 (segment (start 123.95 108.73) (end 125.5 110.28) (width 1) (layer "B.Cu") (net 28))
 (segment (start 136 130.26) (end 143.28 122.98) (width 1) (layer "B.Cu") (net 28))
 (segment (start 143.28 110.28) (end 141.73 111.83) (width 1) (layer "B.Cu") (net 28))
 (segment (start 116.248691 143.716615) (end 116.248691 156.000414) (width 1) (layer "B.Cu") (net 28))
 (segment (start 136 133.414214) (end 136 130.26) (width 1) (layer "B.Cu") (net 28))
 (segment (start 143.28 135.68) (end 141.6 134) (width 1) (layer "B.Cu") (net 28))
 (segment (start 141.73 121.43) (end 143.28 122.98) (width 1) (layer "B.Cu") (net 28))
 (segment (start 141.648691 114.451309) (end 143.28 112.82) (width 0.25) (layer "F.Cu") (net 9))
 (segment (start 141.648691 156.000414) (end 141.648691 114.451309) (width 0.25) (layer "F.Cu") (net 9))
 (segment (start 132.4409 112.205) (end 132.4409 102.1709) (width 0.25) (layer "F.Cu") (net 19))
 (segment (start 122.075 96.425) (end 122.075 105.075) (width 0.25) (layer "F.Cu") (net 19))
 (segment (start 128.948691 147) (end 130.3509 145.597791) (width 0.25) (layer "F.Cu") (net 19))
 (segment (start 122.2 105.2) (end 125.5 105.2) (width 0.25) (layer "F.Cu") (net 19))
 (segment (start 122.075 105.075) (end 122.2 105.2) (width 0.25) (layer "F.Cu") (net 19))
 (segment (start 132.4409 102.1709) (end 126.675 96.405) (width 0.25) (layer "F.Cu") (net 19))
 (segment (start 130.3509 114.295) (end 132.4409 112.205) (width 0.25) (layer "F.Cu") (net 19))
 (segment (start 130.3509 145.597791) (end 130.3509 114.295) (width 0.25) (layer "F.Cu") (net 19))
 (segment (start 122.095 96.405) (end 122.075 96.425) (width 0.25) (layer "F.Cu") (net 19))
 (segment (start 126.675 96.405) (end 122.095 96.405) (width 0.25) (layer "F.Cu") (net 19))
 (segment (start 128.948691 156.000414) (end 128.948691 147) (width 0.25) (layer "F.Cu") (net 19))
 (segment (start 129.9009 102.1709) (end 129.9009 143.142924) (width 0.25) (layer "F.Cu") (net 21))
 (segment (start 122.525 98.945) (end 126.675 98.945) (width 0.25) (layer "F.Cu") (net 21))
 (segment (start 129.9009 143.142924) (end 126.408691 146.635133) (width 0.25) (layer "F.Cu") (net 21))
 (segment (start 122.525 101.295) (end 122.525 98.945) (width 0.25) (layer "F.Cu") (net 21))
 (segment (start 125.5 102.66) (end 124.135 101.295) (width 0.25) (layer "F.Cu") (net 21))
 (segment (start 126.675 98.945) (end 129.9009 102.1709) (width 0.25) (layer "F.Cu") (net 21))
 (segment (start 124.135 101.295) (end 122.525 101.295) (width 0.25) (layer "F.Cu") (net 21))
 (segment (start 126.408691 146.635133) (end 126.408691 156.000414) (width 0.25) (layer "F.Cu") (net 21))
 (segment (start 132.5 112.1459) (end 132.5 103.28) (width 0.25) (layer "B.Cu") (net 18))
 (segment (start 132.5 103.28) (end 143.28 92.5) (width 0.25) (layer "B.Cu") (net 18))
 (segment (start 128.948691 115.697209) (end 132.5 112.1459) (width 0.25) (layer "B.Cu") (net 18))
 (segment (start 128.948691 156.000414) (end 128.948691 115.697209) (width 0.25) (layer "B.Cu") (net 18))
 (segment (start 146.728691 156.000414) (end 146.728691 123.888691) (width 0.25) (layer "B.Cu") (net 4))
 (segment (start 146.728691 123.888691) (end 143.28 120.44) (width 0.25) (layer "B.Cu") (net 4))
 (segment (start 144.188691 156.000414) (end 144.188691 151.250414) (width 0.25) (layer "B.Cu") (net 6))
 (segment (start 144.188691 146.311309) (end 145.5 145) (width 0.25) (layer "B.Cu") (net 6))
 (segment (start 145.5 127.74) (end 143.28 125.52) (width 0.25) (layer "B.Cu") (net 6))
 (segment (start 145.5 145) (end 145.5 127.74) (width 0.25) (layer "B.Cu") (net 6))
 (segment (start 144.188691 156.000414) (end 144.188691 146.311309) (width 0.25) (layer "B.Cu") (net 6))
 (segment (start 137.625 132.741116) (end 137.258884 132.375) (width 0.25) (layer "F.Cu") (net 15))
 (segment (start 137.625 135.723612) (end 137.625 132.741116) (width 0.25) (layer "F.Cu") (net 15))
 (segment (start 137.030608 136.318004) (end 137.625 135.723612) (width 0.25) (layer "F.Cu") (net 15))
 (segment (start 137.258884 132.375) (end 136.741116 132.375) (width 0.25) (layer "F.Cu") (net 15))
 (segment (start 134.028691 135.087425) (end 134.028691 156.000414) (width 0.25) (layer "F.Cu") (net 15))
 (segment (start 136.741116 132.375) (end 134.028691 135.087425) (width 0.25) (layer "F.Cu") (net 15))
 (via (at 137.030608 136.318004) (size 0.6) (drill 0.3) (layers "F.Cu" "B.Cu") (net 15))
 (segment (start 138.318004 136.318004) (end 140.22 138.22) (width 0.25) (layer "B.Cu") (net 15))
 (segment (start 137.030608 136.318004) (end 138.318004 136.318004) (width 0.25) (layer "B.Cu") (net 15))
 (segment (start 140.22 138.22) (end 143.28 138.22) (width 0.25) (layer "B.Cu") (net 15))
 (segment (start 125.5 92.5) (end 127.125 94.125) (width 0.25) (layer "B.Cu") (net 20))
 (segment (start 127.125 94.125) (end 127.125 146.283691) (width 0.25) (layer "B.Cu") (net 20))
 (segment (start 127.125 146.283691) (end 126.408691 147) (width 0.25) (layer "B.Cu") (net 20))
 (segment (start 126.408691 156.000414) (end 126.408691 147) (width 0.25) (layer "B.Cu") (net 20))
 (segment (start 144.455 141.246701) (end 144.455 131.775) (width 0.25) (layer "B.Cu") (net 10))
 (segment (start 144.455 131.775) (end 143.28 130.6) (width 0.25) (layer "B.Cu") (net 10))
 (segment (start 139.108691 156.000414) (end 139.108691 146.59301) (width 0.25) (layer "B.Cu") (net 10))
 (segment (start 139.108691 146.59301) (end 144.455 141.246701) (width 0.25) (layer "B.Cu") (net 10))
 (segment (start 146.255 116.725) (end 144.89 115.36) (width 0.25) (layer "F.Cu") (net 7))
 (segment (start 144.188691 156.000414) (end 144.188691 146.635133) (width 0.25) (layer "F.Cu") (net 7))
 (segment (start 146.255 144.568824) (end 146.255 116.725) (width 0.25) (layer "F.Cu") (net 7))
 (segment (start 144.89 115.36) (end 143.28 115.36) (width 0.25) (layer "F.Cu") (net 7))
 (segment (start 144.188691 146.635133) (end 146.255 144.568824) (width 0.25) (layer "F.Cu") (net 7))
 (segment (start 136.568691 156.000414) (end 136.568691 146.635133) (width 0.25) (layer "F.Cu") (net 13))
 (segment (start 135.69 134.31) (end 137 133) (width 0.25) (layer "F.Cu") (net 13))
 (segment (start 135.69 145.756442) (end 135.69 134.31) (width 0.25) (layer "F.Cu") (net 13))
 (segment (start 136.568691 146.635133) (end 135.69 145.756442) (width 0.25) (layer "F.Cu") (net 13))
 (via (at 137 133) (size 0.6) (drill 0.3) (layers "F.Cu" "B.Cu") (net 13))
 (segment (start 137.14 133.14) (end 137 133) (width 0.25) (layer "B.Cu") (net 13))
 (segment (start 143.28 133.14) (end 137.14 133.14) (width 0.25) (layer "B.Cu") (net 13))
 (segment (start 146.728691 156.000414) (end 146.728691 101.958691) (width 0.25) (layer "F.Cu") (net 5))
 (segment (start 146.728691 101.958691) (end 144.89 100.12) (width 0.25) (layer "F.Cu") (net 5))
 (segment (start 144.89 100.12) (end 143.28 100.12) (width 0.25) (layer "F.Cu") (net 5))
 (segment (start 126.675 145.193691) (end 126.675 96.215) (width 0.25) (layer "B.Cu") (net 22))
 (segment (start 126.675 96.215) (end 125.5 95.04) (width 0.25) (layer "B.Cu") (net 22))
 (segment (start 123.868691 148) (end 126.675 145.193691) (width 0.25) (layer "B.Cu") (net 22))
 (segment (start 123.868691 156.000414) (end 123.868691 148) (width 0.25) (layer "B.Cu") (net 22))
 (segment (start 123.868691 147) (end 127.5509 143.317791) (width 0.25) (layer "F.Cu") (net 23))
 (segment (start 123.868691 156.000414) (end 123.868691 147) (width 0.25) (layer "F.Cu") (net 23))
 (segment (start 127.5509 102.1709) (end 125.5 100.12) (width 0.25) (layer "F.Cu") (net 23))
 (segment (start 127.5509 143.317791) (end 127.5509 102.1709) (width 0.25) (layer "F.Cu") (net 23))
 (segment (start 149.268691 101.958691) (end 146.255 98.945) (width 0.25) (layer "F.Cu") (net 3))
 (segment (start 149.268691 156.000414) (end 149.268691 101.958691) (width 0.25) (layer "F.Cu") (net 3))
 (segment (start 142.105 98.945) (end 142.105 101.485) (width 0.25) (layer "F.Cu") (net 3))
 (segment (start 144.89 102.66) (end 143.28 102.66) (width 0.25) (layer "F.Cu") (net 3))
 (segment (start 142.105 101.485) (end 143.28 102.66) (width 0.25) (layer "F.Cu") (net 3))
 (segment (start 146.255 98.945) (end 142.105 98.945) (width 0.25) (layer "F.Cu") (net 3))
 (segment (start 131.488691 143.511309) (end 131.488691 156.000414) (width 0.25) (layer "B.Cu") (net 16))
 (segment (start 135.69 102.63) (end 135.69 118.81) (width 0.25) (layer "B.Cu") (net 16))
 (segment (start 135.69 118.81) (end 130.39 124.11) (width 0.25) (layer "B.Cu") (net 16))
 (segment (start 130.39 142.412618) (end 131.488691 143.511309) (width 0.25) (layer "B.Cu") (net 16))
 (segment (start 143.28 95.04) (end 135.69 102.63) (width 0.25) (layer "B.Cu") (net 16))
 (segment (start 130.39 124.11) (end 130.39 142.412618) (width 0.25) (layer "B.Cu") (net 16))
 (segment (start 135 111.5) (end 135 101.825) (width 0.25) (layer "F.Cu") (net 17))
 (segment (start 133.09 145.033824) (end 133.09 113.41) (width 0.25) (layer "F.Cu") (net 17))
 (segment (start 122.24 107.74) (end 125.5 107.74) (width 0.25) (layer "F.Cu") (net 17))
 (segment (start 122.825 93.675) (end 121.625 94.875) (width 0.25) (layer "F.Cu") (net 17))
 (segment (start 121.625 107.125) (end 122.24 107.74) (width 0.25) (layer "F.Cu") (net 17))
 (segment (start 121.625 94.875) (end 121.625 107.125) (width 0.25) (layer "F.Cu") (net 17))
 (segment (start 131.488691 146.635133) (end 133.09 145.033824) (width 0.25) (layer "F.Cu") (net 17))
 (segment (start 131.488691 156.000414) (end 131.488691 146.635133) (width 0.25) (layer "F.Cu") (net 17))
 (segment (start 126.85 93.675) (end 122.825 93.675) (width 0.25) (layer "F.Cu") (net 17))
 (segment (start 135 101.825) (end 126.85 93.675) (width 0.25) (layer "F.Cu") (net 17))
 (segment (start 133.09 113.41) (end 135 111.5) (width 0.25) (layer "F.Cu") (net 17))
 (segment (start 138.39 147.61) (end 138.39 107.74) (width 0.25) (layer "F.Cu") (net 12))
 (segment (start 146.278691 104.048691) (end 146.278691 107) (width 0.25) (layer "F.Cu") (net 12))
 (segment (start 145.538691 107.74) (end 143.28 107.74) (width 0.25) (layer "F.Cu") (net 12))
 (segment (start 138 148) (end 138.39 147.61) (width 0.25) (layer "F.Cu") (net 12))
 (segment (start 142.105 104.025) (end 146.255 104.025) (width 0.25) (layer "F.Cu") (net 12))
 (segment (start 146.255 104.025) (end 146.278691 104.048691) (width 0.25) (layer "F.Cu") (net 12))
 (segment (start 138.39 107.74) (end 142.105 104.025) (width 0.25) (layer "F.Cu") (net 12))
 (segment (start 146.278691 107) (end 145.538691 107.74) (width 0.25) (layer "F.Cu") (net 12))
 (via (at 138 148) (size 0.6) (drill 0.3) (layers "F.Cu" "B.Cu") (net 12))
 (segment (start 136.568691 156.000414) (end 136.568691 149.431309) (width 0.25) (layer "B.Cu") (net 12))
 (segment (start 136.568691 156.000414) (end 136.568691 151.250414) (width 0.25) (layer "B.Cu") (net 12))
 (segment (start 136.568691 149.431309) (end 138 148) (width 0.25) (layer "B.Cu") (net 12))
 (segment (start 139.108691 109.371309) (end 143.28 105.2) (width 0.25) (layer "F.Cu") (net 11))
 (segment (start 139.108691 156.000414) (end 139.108691 109.371309) (width 0.25) (layer "F.Cu") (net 11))
 (segment (start 134.028691 156.000414) (end 134.028691 150.011309) (width 0.25) (layer "B.Cu") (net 14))
 (segment (start 134.028691 150.011309) (end 143.28 140.76) (width 0.25) (layer "B.Cu") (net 14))
 (segment (start 141.648691 156.000414) (end 141.648691 147.851309) (width 0.25) (layer "B.Cu") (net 8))
 (segment (start 141.648691 147.851309) (end 145 144.5) (width 0.25) (layer "B.Cu") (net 8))
 (segment (start 145 129.78) (end 143.28 128.06) (width 0.25) (layer "B.Cu") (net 8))
 (segment (start 145 144.5) (end 145 129.78) (width 0.25) (layer "B.Cu") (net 8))
 (segment (start 149.268691 123.888691) (end 143.28 117.9) (width 0.25) (layer "B.Cu") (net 2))
 (segment (start 149.268691 156.000414) (end 149.268691 123.888691) (width 0.25) (layer "B.Cu") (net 2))
 (segment (start 121.328691 124.611309) (end 125.5 120.44) (width 0.25) (layer "B.Cu") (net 24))
 (segment (start 121.328691 156.000414) (end 121.328691 124.611309) (width 0.25) (layer "B.Cu") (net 24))
 (segment (start 112.305212 122.305212) (end 112.305212 139.516521) (width 0.25) (layer "F.Cu") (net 27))
 (segment (start 118.788691 156.000414) (end 118.788691 146.635133) (width 0.25) (layer "F.Cu") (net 27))
 (segment (start 112.305212 139.516521) (end 118.788691 146) (width 0.25) (layer "F.Cu") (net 27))
 (segment (start 111.5 121.5) (end 112.305212 122.305212) (width 0.25) (layer "F.Cu") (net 27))
 (segment (start 118.788691 146.635133) (end 118.788691 146) (width 0.25) (layer "F.Cu") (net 27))
 (via (at 111.5 121.5) (size 0.6) (drill 0.3) (layers "F.Cu" "B.Cu") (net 27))
 (segment (start 115.1 117.9) (end 111.5 121.5) (width 0.25) (layer "B.Cu") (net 27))
 (segment (start 125.5 117.9) (end 115.1 117.9) (width 0.25) (layer "B.Cu") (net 27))
 (segment (start 118.788691 156.000414) (end 118.788691 129.672575) (width 0.25) (layer "B.Cu") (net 26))
 (segment (start 110.875 121.758884) (end 110.875 121.125) (width 0.25) (layer "B.Cu") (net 26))
 (segment (start 110.875 121.125) (end 119.18 112.82) (width 0.25) (layer "B.Cu") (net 26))
 (segment (start 118.788691 129.672575) (end 110.875 121.758884) (width 0.25) (layer "B.Cu") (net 26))
 (segment (start 119.18 112.82) (end 125.5 112.82) (width 0.25) (layer "B.Cu") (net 26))
 (segment (start 127 141.61) (end 121.328691 147.281309) (width 0.25) (layer "F.Cu") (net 25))
 (segment (start 121.328691 147.281309) (end 121.328691 156.000414) (width 0.25) (layer "F.Cu") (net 25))
 (segment (start 127 127.02) (end 127 141.61) (width 0.25) (layer "F.Cu") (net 25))
 (segment (start 125.5 125.52) (end 127 127.02) (width 0.25) (layer "F.Cu") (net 25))
 (segment (start 125.5 138.22) (end 116.1 138.22) (width 1) (layer "F.Cu") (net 37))
 (segment (start 125.460479 138.180479) (end 125.5 138.22) (width 1) (layer "F.Cu") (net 37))
 (segment (start 116.1 138.22) (end 116 138.12) (width 1) (layer "F.Cu") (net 37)))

